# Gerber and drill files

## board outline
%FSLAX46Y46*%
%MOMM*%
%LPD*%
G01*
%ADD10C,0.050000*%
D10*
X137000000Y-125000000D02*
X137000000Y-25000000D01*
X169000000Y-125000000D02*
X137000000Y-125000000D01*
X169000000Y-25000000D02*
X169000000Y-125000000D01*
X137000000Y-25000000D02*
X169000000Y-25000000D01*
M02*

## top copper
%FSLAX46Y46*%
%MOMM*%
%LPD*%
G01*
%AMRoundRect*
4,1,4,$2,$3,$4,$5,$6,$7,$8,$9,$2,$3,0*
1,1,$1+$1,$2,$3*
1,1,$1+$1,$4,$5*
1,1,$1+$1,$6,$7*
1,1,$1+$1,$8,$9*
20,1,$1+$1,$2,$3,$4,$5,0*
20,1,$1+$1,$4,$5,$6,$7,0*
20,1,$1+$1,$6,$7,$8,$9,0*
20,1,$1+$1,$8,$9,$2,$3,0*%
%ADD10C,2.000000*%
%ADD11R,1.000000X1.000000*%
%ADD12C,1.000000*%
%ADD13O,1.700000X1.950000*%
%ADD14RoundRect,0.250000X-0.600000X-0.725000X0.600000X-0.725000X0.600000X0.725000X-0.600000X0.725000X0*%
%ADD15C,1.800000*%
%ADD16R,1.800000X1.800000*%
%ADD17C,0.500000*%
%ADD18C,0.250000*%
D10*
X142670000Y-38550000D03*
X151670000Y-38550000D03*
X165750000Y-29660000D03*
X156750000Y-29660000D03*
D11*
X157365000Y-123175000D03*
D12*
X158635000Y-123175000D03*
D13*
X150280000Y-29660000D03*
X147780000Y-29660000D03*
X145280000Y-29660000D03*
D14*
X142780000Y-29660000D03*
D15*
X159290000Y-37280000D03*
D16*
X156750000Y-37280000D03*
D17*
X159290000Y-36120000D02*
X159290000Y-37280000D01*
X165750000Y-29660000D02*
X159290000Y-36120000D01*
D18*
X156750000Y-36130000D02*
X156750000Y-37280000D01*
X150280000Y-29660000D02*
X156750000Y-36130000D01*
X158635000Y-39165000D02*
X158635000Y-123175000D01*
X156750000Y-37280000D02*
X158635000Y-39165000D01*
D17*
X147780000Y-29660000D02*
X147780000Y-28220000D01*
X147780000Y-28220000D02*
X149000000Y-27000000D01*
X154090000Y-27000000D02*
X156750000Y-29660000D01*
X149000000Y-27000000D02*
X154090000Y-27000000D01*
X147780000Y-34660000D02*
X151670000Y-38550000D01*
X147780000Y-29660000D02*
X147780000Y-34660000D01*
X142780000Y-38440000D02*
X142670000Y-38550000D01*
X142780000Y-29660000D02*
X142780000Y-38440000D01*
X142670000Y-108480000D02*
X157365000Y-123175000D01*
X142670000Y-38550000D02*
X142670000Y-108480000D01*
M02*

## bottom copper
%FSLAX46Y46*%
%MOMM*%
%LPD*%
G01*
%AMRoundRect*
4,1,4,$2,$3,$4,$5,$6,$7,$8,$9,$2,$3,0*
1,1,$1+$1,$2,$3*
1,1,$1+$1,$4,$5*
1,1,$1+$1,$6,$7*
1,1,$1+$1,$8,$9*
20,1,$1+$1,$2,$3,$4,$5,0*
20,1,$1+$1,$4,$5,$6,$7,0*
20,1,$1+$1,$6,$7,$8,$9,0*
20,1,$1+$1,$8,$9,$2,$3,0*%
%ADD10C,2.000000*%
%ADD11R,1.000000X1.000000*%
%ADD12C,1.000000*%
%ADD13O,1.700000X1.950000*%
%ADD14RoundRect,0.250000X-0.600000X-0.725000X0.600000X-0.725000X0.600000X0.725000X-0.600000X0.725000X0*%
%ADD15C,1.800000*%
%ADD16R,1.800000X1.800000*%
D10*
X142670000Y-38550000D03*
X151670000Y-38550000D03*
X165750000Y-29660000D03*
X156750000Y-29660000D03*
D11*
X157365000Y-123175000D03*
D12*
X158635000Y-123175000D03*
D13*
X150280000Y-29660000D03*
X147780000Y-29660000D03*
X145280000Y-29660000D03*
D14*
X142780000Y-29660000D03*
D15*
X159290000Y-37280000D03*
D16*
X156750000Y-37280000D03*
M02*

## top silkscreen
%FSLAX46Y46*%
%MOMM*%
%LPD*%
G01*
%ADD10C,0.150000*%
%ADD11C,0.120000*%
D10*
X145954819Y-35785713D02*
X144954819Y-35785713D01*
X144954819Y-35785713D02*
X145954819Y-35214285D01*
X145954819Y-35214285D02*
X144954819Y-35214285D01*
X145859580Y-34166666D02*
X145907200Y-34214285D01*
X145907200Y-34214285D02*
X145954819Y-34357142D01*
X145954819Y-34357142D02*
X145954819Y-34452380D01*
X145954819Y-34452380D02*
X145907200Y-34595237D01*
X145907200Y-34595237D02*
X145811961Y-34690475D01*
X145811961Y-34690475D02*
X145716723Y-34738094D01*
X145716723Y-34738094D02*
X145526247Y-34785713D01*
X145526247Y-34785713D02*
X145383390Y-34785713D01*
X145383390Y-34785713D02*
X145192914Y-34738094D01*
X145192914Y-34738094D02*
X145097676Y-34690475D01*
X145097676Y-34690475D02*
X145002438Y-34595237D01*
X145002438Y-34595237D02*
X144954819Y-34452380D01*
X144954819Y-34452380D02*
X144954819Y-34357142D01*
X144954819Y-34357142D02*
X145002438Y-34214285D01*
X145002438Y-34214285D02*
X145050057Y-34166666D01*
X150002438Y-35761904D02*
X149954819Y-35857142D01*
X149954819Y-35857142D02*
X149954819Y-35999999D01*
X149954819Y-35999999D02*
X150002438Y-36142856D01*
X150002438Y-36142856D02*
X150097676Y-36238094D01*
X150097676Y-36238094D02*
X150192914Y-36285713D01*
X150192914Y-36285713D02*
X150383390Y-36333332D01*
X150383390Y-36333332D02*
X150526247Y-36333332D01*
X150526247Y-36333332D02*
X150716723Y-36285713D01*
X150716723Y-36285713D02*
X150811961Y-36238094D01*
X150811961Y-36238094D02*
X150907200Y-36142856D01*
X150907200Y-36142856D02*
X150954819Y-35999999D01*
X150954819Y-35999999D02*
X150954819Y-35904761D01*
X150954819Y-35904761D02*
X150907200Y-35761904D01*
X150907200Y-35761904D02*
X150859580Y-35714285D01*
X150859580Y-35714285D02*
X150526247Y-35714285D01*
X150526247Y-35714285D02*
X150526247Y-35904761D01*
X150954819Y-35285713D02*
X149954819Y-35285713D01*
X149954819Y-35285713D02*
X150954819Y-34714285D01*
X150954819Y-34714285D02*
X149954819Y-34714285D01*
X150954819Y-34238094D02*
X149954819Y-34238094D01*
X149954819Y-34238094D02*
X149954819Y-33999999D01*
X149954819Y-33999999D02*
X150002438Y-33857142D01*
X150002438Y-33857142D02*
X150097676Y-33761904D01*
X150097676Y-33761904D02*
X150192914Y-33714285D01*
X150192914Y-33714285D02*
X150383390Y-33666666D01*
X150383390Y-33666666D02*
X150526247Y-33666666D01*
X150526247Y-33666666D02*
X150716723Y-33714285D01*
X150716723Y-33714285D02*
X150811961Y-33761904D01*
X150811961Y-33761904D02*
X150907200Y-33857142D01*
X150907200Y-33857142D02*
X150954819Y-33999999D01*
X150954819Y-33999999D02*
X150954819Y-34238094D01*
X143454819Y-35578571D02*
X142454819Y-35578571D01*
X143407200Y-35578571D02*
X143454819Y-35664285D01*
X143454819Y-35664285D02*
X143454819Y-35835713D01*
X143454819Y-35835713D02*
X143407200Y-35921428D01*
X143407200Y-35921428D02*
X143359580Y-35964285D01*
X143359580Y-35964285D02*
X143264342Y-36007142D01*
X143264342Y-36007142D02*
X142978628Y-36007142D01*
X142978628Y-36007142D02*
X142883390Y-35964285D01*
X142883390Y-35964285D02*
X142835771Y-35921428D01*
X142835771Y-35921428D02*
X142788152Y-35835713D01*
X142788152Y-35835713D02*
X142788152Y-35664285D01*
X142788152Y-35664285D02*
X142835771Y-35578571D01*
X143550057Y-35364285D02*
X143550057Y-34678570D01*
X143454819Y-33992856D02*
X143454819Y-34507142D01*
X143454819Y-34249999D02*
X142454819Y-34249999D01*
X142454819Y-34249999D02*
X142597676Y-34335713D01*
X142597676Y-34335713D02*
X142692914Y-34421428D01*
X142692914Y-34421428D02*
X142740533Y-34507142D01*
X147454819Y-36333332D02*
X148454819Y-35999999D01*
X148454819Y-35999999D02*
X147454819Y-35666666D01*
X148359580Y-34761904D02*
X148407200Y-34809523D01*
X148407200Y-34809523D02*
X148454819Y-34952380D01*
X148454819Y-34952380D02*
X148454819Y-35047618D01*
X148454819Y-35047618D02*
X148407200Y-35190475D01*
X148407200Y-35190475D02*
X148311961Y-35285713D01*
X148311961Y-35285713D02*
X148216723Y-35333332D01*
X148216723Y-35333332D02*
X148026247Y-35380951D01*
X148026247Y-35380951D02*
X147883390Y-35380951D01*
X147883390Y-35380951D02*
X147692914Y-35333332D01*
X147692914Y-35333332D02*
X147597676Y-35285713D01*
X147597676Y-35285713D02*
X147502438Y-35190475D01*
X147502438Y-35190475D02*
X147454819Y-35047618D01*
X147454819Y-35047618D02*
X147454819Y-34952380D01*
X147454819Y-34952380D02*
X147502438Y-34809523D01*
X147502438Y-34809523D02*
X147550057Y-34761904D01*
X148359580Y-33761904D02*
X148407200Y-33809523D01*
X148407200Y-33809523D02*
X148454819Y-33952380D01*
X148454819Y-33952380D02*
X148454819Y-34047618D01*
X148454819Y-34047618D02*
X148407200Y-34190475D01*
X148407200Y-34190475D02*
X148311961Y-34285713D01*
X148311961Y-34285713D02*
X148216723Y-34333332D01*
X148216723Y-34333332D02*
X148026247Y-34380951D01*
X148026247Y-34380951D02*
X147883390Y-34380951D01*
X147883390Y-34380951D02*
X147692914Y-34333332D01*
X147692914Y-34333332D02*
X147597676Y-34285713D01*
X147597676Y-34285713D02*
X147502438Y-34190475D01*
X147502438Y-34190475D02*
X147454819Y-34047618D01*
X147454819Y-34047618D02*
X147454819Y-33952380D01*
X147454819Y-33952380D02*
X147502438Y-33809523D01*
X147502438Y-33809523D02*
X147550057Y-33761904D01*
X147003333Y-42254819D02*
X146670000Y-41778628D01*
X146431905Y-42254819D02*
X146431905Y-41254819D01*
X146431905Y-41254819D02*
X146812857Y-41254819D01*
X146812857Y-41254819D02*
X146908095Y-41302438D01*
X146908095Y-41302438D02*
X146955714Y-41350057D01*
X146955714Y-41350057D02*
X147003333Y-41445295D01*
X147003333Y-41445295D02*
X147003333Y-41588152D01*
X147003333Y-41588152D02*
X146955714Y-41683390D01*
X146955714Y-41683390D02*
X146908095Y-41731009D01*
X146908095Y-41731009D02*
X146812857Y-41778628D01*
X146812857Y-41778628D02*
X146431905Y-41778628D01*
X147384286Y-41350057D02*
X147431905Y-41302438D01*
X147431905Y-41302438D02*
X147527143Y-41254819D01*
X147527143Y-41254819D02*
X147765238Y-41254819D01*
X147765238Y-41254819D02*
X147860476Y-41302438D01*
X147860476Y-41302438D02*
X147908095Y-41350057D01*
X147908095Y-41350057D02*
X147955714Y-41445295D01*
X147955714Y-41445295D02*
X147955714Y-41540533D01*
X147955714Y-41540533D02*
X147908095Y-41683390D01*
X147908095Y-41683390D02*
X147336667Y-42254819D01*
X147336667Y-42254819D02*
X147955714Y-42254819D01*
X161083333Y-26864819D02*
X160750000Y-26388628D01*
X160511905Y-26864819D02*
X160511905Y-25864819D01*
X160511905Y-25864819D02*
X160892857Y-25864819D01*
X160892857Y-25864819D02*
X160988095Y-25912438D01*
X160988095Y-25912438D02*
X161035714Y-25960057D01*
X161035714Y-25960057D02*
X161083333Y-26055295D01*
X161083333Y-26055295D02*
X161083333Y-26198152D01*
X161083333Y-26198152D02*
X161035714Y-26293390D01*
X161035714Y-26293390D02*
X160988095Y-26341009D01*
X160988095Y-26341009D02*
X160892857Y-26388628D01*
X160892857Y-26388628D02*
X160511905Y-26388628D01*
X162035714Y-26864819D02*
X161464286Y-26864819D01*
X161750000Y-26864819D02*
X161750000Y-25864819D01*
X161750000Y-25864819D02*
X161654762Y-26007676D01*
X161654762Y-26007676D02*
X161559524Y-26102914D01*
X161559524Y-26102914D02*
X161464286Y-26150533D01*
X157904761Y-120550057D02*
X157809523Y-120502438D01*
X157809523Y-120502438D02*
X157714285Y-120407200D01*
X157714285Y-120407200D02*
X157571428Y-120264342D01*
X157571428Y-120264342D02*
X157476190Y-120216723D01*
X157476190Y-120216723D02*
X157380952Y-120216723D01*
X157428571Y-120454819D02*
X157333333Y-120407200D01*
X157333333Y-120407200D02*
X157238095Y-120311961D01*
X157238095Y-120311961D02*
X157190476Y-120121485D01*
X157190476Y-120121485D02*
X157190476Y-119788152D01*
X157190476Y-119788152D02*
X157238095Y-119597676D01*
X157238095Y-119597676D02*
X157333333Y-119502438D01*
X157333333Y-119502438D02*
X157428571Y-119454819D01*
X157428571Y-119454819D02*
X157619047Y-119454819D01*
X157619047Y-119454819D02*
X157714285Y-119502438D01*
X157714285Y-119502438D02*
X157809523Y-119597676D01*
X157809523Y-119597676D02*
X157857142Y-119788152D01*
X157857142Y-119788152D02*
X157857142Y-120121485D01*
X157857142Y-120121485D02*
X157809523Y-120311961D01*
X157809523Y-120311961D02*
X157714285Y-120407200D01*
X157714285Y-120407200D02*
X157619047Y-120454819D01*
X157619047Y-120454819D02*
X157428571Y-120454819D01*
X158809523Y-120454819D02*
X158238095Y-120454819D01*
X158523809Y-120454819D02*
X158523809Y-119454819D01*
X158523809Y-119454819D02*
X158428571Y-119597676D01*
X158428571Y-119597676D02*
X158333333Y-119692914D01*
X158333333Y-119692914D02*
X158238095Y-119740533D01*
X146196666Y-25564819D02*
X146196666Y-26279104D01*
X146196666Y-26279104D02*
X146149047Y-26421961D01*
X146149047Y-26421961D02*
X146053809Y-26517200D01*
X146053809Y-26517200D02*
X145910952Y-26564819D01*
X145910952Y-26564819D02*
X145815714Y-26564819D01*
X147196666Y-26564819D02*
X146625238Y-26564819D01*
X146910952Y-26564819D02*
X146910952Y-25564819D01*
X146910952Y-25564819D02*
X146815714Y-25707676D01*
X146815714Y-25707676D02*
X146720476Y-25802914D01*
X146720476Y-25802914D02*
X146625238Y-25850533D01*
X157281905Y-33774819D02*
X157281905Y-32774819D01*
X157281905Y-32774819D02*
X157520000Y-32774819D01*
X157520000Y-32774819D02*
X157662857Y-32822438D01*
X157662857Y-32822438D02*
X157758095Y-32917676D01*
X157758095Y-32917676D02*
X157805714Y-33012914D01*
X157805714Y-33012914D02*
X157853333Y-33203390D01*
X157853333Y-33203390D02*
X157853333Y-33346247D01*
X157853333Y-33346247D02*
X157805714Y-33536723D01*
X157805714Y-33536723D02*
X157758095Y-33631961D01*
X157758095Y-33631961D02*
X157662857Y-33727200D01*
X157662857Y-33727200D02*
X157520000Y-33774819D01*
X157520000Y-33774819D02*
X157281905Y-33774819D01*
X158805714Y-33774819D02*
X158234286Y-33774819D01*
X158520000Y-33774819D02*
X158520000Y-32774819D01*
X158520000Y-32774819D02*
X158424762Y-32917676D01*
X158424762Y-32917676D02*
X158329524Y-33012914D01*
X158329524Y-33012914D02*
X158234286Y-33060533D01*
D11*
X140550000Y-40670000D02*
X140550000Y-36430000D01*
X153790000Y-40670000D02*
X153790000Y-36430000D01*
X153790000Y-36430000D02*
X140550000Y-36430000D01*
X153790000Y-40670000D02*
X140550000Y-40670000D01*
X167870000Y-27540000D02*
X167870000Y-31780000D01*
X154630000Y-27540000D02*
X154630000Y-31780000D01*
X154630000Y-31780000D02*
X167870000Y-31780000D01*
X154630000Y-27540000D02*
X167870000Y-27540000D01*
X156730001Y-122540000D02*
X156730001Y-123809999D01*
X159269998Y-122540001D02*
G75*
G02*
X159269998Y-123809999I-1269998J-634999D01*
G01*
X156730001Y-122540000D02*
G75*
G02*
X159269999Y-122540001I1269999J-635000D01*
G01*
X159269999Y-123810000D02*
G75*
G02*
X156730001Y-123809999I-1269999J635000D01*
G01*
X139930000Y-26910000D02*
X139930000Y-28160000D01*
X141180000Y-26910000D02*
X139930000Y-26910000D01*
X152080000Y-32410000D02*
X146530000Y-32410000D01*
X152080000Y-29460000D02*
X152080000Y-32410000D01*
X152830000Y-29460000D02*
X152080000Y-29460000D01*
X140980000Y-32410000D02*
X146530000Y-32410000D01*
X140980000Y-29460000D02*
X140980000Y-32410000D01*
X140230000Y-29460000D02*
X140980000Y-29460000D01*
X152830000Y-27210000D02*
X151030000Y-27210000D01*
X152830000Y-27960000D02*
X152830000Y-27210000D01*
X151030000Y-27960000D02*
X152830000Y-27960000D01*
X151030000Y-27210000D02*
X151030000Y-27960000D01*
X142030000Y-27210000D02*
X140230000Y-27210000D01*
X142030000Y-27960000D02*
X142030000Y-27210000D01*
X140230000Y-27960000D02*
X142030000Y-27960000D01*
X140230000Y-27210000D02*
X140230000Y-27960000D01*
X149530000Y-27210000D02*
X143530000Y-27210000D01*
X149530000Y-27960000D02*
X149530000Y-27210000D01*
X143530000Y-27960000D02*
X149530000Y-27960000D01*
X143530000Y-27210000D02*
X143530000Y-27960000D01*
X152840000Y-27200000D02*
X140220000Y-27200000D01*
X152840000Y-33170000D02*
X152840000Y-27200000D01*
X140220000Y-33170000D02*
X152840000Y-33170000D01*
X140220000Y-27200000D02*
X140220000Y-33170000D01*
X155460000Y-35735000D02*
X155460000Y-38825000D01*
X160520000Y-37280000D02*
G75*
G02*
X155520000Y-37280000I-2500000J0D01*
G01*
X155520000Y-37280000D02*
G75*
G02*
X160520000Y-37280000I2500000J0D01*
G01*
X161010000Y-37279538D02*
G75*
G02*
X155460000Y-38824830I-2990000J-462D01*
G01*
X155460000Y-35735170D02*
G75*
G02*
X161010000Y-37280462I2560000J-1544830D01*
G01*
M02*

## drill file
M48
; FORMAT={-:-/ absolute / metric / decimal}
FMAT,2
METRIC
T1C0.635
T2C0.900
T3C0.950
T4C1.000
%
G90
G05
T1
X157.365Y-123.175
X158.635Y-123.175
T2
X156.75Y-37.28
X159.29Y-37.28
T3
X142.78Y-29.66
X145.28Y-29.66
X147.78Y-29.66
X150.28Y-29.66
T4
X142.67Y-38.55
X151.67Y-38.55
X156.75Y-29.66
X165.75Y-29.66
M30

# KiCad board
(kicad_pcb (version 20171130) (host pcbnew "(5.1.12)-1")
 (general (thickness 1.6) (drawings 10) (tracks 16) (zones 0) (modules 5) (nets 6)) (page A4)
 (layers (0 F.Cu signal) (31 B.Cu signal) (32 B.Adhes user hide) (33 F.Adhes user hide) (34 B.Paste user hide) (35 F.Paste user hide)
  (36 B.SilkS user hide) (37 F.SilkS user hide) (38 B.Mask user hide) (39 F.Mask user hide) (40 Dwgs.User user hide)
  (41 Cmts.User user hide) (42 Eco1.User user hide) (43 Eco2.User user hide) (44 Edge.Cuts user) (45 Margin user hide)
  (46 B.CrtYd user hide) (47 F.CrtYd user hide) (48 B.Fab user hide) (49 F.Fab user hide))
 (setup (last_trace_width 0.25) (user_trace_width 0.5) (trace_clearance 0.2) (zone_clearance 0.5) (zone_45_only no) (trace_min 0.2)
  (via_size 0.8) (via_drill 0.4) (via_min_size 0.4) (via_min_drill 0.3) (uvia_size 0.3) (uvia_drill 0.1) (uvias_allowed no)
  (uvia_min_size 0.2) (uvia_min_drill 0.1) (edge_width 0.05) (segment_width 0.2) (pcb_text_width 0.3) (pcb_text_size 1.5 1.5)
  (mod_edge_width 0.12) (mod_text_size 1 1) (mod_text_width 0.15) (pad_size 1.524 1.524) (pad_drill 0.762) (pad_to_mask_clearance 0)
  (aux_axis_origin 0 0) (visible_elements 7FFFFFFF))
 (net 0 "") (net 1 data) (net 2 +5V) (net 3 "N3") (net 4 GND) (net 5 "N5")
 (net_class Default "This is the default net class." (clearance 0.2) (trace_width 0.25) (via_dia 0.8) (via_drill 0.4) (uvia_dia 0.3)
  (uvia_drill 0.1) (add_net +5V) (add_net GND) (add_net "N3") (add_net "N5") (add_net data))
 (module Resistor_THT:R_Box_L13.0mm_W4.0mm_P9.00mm (layer F.Cu) (at 151.67 38.55 180)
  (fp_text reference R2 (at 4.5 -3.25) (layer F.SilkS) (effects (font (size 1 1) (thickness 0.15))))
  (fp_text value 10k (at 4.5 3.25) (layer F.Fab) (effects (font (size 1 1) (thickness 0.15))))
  (fp_line (start 11.12 -2.12) (end 11.12 2.12) (layer F.SilkS) (width 0.12))
  (fp_line (start -2.12 -2.12) (end -2.12 2.12) (layer F.SilkS) (width 0.12))
  (fp_line (start -2.12 2.12) (end 11.12 2.12) (layer F.SilkS) (width 0.12))
  (fp_line (start -2.12 -2.12) (end 11.12 -2.12) (layer F.SilkS) (width 0.12))
  (pad 2 thru_hole circle (at 9 0 180) (size 2 2) (drill 1) (layers *.Cu *.Mask) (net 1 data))
  (pad 1 thru_hole circle (at 0 0 180) (size 2 2) (drill 1) (layers *.Cu *.Mask) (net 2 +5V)))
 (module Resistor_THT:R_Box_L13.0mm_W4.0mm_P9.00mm (layer F.Cu) (at 156.75 29.66)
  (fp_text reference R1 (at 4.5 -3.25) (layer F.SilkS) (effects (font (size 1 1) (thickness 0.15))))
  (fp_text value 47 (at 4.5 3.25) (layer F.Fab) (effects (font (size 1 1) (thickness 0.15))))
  (fp_line (start 11.12 -2.12) (end 11.12 2.12) (layer F.SilkS) (width 0.12))
  (fp_line (start -2.12 -2.12) (end -2.12 2.12) (layer F.SilkS) (width 0.12))
  (fp_line (start -2.12 2.12) (end 11.12 2.12) (layer F.SilkS) (width 0.12))
  (fp_line (start -2.12 -2.12) (end 11.12 -2.12) (layer F.SilkS) (width 0.12))
  (pad 2 thru_hole circle (at 9 0) (size 2 2) (drill 1) (layers *.Cu *.Mask) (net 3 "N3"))
  (pad 1 thru_hole circle (at 0 0) (size 2 2) (drill 1) (layers *.Cu *.Mask) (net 2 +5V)))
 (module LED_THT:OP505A (layer F.Cu) (at 158 120)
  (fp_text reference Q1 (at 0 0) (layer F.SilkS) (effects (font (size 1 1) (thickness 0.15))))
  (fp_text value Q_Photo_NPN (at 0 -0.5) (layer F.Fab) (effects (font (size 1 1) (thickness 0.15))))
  (fp_line (start -1.269999 2.54) (end -1.269999 3.809999) (layer F.SilkS) (width 0.12))
  (fp_arc (start 0 3.175) (end 1.269998 3.809999) (angle -53.13010235) (layer F.SilkS) (width 0.12))
  (fp_arc (start 0 3.175) (end 1.269999 2.540001) (angle -126.8698976) (layer F.SilkS) (width 0.12))
  (fp_arc (start 0 3.175) (end -1.269999 3.809999) (angle -126.8698976) (layer F.SilkS) (width 0.12))
  (pad 1 thru_hole rect (at -0.635 3.175) (size 1 1) (drill 0.635) (layers *.Cu *.Mask) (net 1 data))
  (pad 2 thru_hole circle (at 0.635 3.175) (size 1 1) (drill 0.635) (layers *.Cu *.Mask) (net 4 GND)))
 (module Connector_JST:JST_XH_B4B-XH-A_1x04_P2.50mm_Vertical (layer F.Cu) (at 142.78 29.66)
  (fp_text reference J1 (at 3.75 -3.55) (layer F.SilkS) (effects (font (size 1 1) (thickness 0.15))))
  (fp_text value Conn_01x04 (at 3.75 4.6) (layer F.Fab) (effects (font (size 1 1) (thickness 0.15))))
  (fp_line (start -2.85 -2.75) (end -2.85 -1.5) (layer F.SilkS) (width 0.12))
  (fp_line (start -1.6 -2.75) (end -2.85 -2.75) (layer F.SilkS) (width 0.12))
  (fp_line (start 9.3 2.75) (end 3.75 2.75) (layer F.SilkS) (width 0.12))
  (fp_line (start 9.3 -0.2) (end 9.3 2.75) (layer F.SilkS) (width 0.12))
  (fp_line (start 10.05 -0.2) (end 9.3 -0.2) (layer F.SilkS) (width 0.12))
  (fp_line (start -1.8 2.75) (end 3.75 2.75) (layer F.SilkS) (width 0.12))
  (fp_line (start -1.8 -0.2) (end -1.8 2.75) (layer F.SilkS) (width 0.12))
  (fp_line (start -2.55 -0.2) (end -1.8 -0.2) (layer F.SilkS) (width 0.12))
  (fp_line (start 10.05 -2.45) (end 8.25 -2.45) (layer F.SilkS) (width 0.12))
  (fp_line (start 10.05 -1.7) (end 10.05 -2.45) (layer F.SilkS) (width 0.12))
  (fp_line (start 8.25 -1.7) (end 10.05 -1.7) (layer F.SilkS) (width 0.12))
  (fp_line (start 8.25 -2.45) (end 8.25 -1.7) (layer F.SilkS) (width 0.12))
  (fp_line (start -0.75 -2.45) (end -2.55 -2.45) (layer F.SilkS) (width 0.12))
  (fp_line (start -0.75 -1.7) (end -0.75 -2.45) (layer F.SilkS) (width 0.12))
  (fp_line (start -2.55 -1.7) (end -0.75 -1.7) (layer F.SilkS) (width 0.12))
  (fp_line (start -2.55 -2.45) (end -2.55 -1.7) (layer F.SilkS) (width 0.12))
  (fp_line (start 6.75 -2.45) (end 0.75 -2.45) (layer F.SilkS) (width 0.12))
  (fp_line (start 6.75 -1.7) (end 6.75 -2.45) (layer F.SilkS) (width 0.12))
  (fp_line (start 0.75 -1.7) (end 6.75 -1.7) (layer F.SilkS) (width 0.12))
  (fp_line (start 0.75 -2.45) (end 0.75 -1.7) (layer F.SilkS) (width 0.12))
  (fp_line (start 10.06 -2.46) (end -2.56 -2.46) (layer F.SilkS) (width 0.12))
  (fp_line (start 10.06 3.51) (end 10.06 -2.46) (layer F.SilkS) (width 0.12))
  (fp_line (start -2.56 3.51) (end 10.06 3.51) (layer F.SilkS) (width 0.12))
  (fp_line (start -2.56 -2.46) (end -2.56 3.51) (layer F.SilkS) (width 0.12))
  (pad 4 thru_hole oval (at 7.5 0) (size 1.7 1.95) (drill 0.95) (layers *.Cu *.Mask) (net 4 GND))
  (pad 3 thru_hole oval (at 5 0) (size 1.7 1.95) (drill 0.95) (layers *.Cu *.Mask) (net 2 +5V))
  (pad 2 thru_hole oval (at 2.5 0) (size 1.7 1.95) (drill 0.95) (layers *.Cu *.Mask) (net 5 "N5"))
  (pad 1 thru_hole roundrect (at 0 0) (size 1.7 1.95) (drill 0.95) (layers *.Cu *.Mask) (roundrect_rratio 0.1470588235294118) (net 1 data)))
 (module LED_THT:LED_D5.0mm (layer F.Cu) (at 156.75 37.28)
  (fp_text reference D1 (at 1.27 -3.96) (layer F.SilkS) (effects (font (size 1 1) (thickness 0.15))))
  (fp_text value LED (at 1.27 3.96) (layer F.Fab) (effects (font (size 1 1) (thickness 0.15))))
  (fp_line (start -1.29 -1.545) (end -1.29 1.545) (layer F.SilkS) (width 0.12))
  (fp_circle (center 1.27 0) (end 3.77 0) (layer F.SilkS) (width 0.12))
  (fp_arc (start 1.27 0) (end -1.29 1.54483) (angle -148.9) (layer F.SilkS) (width 0.12))
  (fp_arc (start 1.27 0) (end -1.29 -1.54483) (angle 148.9) (layer F.SilkS) (width 0.12))
  (pad 2 thru_hole circle (at 2.54 0) (size 1.8 1.8) (drill 0.9) (layers *.Cu *.Mask) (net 3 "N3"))
  (pad 1 thru_hole rect (at 0 0) (size 1.8 1.8) (drill 0.9) (layers *.Cu *.Mask) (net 4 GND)))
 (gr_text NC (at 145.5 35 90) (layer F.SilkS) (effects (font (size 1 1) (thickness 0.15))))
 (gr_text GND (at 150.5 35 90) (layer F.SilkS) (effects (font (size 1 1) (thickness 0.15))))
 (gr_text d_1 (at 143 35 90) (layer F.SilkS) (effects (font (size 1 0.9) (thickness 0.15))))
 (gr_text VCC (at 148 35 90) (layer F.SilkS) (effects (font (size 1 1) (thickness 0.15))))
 (gr_line (start 137 125) (end 137 25) (layer Edge.Cuts) (width 0.05))
 (gr_line (start 169 125) (end 137 125) (layer Edge.Cuts) (width 0.05))
 (gr_line (start 169 25) (end 169 125) (layer Edge.Cuts) (width 0.05))
 (gr_line (start 137 25) (end 169 25) (layer Edge.Cuts) (width 0.05))
 (segment (start 159.29 36.12) (end 159.29 37.28) (width 0.5) (layer F.Cu) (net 3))
 (segment (start 165.75 29.66) (end 159.29 36.12) (width 0.5) (layer F.Cu) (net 3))
 (segment (start 156.75 36.13) (end 156.75 37.28) (width 0.25) (layer F.Cu) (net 4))
 (segment (start 150.28 29.66) (end 156.75 36.13) (width 0.25) (layer F.Cu) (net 4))
 (segment (start 158.635 39.165) (end 158.635 123.175) (width 0.25) (layer F.Cu) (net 4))
 (segment (start 156.75 37.28) (end 158.635 39.165) (width 0.25) (layer F.Cu) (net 4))
 (segment (start 147.78 29.66) (end 147.78 28.22) (width 0.5) (layer F.Cu) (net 2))
 (segment (start 147.78 28.22) (end 149 27) (width 0.5) (layer F.Cu) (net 2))
 (segment (start 154.09 27) (end 156.75 29.66) (width 0.5) (layer F.Cu) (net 2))
 (segment (start 149 27) (end 154.09 27) (width 0.5) (layer F.Cu) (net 2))
 (segment (start 147.78 34.66) (end 151.67 38.55) (width 0.5) (layer F.Cu) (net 2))
 (segment (start 147.78 29.66) (end 147.78 34.66) (width 0.5) (layer F.Cu) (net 2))
 (segment (start 142.78 38.44) (end 142.67 38.55) (width 0.5) (layer F.Cu) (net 1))
 (segment (start 142.78 29.66) (end 142.78 38.44) (width 0.5) (layer F.Cu) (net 1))
 (segment (start 142.67 108.48) (end 157.365 123.175) (width 0.5) (layer F.Cu) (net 1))
 (segment (start 142.67 38.55) (end 142.67 108.48) (width 0.5) (layer F.Cu) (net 1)))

